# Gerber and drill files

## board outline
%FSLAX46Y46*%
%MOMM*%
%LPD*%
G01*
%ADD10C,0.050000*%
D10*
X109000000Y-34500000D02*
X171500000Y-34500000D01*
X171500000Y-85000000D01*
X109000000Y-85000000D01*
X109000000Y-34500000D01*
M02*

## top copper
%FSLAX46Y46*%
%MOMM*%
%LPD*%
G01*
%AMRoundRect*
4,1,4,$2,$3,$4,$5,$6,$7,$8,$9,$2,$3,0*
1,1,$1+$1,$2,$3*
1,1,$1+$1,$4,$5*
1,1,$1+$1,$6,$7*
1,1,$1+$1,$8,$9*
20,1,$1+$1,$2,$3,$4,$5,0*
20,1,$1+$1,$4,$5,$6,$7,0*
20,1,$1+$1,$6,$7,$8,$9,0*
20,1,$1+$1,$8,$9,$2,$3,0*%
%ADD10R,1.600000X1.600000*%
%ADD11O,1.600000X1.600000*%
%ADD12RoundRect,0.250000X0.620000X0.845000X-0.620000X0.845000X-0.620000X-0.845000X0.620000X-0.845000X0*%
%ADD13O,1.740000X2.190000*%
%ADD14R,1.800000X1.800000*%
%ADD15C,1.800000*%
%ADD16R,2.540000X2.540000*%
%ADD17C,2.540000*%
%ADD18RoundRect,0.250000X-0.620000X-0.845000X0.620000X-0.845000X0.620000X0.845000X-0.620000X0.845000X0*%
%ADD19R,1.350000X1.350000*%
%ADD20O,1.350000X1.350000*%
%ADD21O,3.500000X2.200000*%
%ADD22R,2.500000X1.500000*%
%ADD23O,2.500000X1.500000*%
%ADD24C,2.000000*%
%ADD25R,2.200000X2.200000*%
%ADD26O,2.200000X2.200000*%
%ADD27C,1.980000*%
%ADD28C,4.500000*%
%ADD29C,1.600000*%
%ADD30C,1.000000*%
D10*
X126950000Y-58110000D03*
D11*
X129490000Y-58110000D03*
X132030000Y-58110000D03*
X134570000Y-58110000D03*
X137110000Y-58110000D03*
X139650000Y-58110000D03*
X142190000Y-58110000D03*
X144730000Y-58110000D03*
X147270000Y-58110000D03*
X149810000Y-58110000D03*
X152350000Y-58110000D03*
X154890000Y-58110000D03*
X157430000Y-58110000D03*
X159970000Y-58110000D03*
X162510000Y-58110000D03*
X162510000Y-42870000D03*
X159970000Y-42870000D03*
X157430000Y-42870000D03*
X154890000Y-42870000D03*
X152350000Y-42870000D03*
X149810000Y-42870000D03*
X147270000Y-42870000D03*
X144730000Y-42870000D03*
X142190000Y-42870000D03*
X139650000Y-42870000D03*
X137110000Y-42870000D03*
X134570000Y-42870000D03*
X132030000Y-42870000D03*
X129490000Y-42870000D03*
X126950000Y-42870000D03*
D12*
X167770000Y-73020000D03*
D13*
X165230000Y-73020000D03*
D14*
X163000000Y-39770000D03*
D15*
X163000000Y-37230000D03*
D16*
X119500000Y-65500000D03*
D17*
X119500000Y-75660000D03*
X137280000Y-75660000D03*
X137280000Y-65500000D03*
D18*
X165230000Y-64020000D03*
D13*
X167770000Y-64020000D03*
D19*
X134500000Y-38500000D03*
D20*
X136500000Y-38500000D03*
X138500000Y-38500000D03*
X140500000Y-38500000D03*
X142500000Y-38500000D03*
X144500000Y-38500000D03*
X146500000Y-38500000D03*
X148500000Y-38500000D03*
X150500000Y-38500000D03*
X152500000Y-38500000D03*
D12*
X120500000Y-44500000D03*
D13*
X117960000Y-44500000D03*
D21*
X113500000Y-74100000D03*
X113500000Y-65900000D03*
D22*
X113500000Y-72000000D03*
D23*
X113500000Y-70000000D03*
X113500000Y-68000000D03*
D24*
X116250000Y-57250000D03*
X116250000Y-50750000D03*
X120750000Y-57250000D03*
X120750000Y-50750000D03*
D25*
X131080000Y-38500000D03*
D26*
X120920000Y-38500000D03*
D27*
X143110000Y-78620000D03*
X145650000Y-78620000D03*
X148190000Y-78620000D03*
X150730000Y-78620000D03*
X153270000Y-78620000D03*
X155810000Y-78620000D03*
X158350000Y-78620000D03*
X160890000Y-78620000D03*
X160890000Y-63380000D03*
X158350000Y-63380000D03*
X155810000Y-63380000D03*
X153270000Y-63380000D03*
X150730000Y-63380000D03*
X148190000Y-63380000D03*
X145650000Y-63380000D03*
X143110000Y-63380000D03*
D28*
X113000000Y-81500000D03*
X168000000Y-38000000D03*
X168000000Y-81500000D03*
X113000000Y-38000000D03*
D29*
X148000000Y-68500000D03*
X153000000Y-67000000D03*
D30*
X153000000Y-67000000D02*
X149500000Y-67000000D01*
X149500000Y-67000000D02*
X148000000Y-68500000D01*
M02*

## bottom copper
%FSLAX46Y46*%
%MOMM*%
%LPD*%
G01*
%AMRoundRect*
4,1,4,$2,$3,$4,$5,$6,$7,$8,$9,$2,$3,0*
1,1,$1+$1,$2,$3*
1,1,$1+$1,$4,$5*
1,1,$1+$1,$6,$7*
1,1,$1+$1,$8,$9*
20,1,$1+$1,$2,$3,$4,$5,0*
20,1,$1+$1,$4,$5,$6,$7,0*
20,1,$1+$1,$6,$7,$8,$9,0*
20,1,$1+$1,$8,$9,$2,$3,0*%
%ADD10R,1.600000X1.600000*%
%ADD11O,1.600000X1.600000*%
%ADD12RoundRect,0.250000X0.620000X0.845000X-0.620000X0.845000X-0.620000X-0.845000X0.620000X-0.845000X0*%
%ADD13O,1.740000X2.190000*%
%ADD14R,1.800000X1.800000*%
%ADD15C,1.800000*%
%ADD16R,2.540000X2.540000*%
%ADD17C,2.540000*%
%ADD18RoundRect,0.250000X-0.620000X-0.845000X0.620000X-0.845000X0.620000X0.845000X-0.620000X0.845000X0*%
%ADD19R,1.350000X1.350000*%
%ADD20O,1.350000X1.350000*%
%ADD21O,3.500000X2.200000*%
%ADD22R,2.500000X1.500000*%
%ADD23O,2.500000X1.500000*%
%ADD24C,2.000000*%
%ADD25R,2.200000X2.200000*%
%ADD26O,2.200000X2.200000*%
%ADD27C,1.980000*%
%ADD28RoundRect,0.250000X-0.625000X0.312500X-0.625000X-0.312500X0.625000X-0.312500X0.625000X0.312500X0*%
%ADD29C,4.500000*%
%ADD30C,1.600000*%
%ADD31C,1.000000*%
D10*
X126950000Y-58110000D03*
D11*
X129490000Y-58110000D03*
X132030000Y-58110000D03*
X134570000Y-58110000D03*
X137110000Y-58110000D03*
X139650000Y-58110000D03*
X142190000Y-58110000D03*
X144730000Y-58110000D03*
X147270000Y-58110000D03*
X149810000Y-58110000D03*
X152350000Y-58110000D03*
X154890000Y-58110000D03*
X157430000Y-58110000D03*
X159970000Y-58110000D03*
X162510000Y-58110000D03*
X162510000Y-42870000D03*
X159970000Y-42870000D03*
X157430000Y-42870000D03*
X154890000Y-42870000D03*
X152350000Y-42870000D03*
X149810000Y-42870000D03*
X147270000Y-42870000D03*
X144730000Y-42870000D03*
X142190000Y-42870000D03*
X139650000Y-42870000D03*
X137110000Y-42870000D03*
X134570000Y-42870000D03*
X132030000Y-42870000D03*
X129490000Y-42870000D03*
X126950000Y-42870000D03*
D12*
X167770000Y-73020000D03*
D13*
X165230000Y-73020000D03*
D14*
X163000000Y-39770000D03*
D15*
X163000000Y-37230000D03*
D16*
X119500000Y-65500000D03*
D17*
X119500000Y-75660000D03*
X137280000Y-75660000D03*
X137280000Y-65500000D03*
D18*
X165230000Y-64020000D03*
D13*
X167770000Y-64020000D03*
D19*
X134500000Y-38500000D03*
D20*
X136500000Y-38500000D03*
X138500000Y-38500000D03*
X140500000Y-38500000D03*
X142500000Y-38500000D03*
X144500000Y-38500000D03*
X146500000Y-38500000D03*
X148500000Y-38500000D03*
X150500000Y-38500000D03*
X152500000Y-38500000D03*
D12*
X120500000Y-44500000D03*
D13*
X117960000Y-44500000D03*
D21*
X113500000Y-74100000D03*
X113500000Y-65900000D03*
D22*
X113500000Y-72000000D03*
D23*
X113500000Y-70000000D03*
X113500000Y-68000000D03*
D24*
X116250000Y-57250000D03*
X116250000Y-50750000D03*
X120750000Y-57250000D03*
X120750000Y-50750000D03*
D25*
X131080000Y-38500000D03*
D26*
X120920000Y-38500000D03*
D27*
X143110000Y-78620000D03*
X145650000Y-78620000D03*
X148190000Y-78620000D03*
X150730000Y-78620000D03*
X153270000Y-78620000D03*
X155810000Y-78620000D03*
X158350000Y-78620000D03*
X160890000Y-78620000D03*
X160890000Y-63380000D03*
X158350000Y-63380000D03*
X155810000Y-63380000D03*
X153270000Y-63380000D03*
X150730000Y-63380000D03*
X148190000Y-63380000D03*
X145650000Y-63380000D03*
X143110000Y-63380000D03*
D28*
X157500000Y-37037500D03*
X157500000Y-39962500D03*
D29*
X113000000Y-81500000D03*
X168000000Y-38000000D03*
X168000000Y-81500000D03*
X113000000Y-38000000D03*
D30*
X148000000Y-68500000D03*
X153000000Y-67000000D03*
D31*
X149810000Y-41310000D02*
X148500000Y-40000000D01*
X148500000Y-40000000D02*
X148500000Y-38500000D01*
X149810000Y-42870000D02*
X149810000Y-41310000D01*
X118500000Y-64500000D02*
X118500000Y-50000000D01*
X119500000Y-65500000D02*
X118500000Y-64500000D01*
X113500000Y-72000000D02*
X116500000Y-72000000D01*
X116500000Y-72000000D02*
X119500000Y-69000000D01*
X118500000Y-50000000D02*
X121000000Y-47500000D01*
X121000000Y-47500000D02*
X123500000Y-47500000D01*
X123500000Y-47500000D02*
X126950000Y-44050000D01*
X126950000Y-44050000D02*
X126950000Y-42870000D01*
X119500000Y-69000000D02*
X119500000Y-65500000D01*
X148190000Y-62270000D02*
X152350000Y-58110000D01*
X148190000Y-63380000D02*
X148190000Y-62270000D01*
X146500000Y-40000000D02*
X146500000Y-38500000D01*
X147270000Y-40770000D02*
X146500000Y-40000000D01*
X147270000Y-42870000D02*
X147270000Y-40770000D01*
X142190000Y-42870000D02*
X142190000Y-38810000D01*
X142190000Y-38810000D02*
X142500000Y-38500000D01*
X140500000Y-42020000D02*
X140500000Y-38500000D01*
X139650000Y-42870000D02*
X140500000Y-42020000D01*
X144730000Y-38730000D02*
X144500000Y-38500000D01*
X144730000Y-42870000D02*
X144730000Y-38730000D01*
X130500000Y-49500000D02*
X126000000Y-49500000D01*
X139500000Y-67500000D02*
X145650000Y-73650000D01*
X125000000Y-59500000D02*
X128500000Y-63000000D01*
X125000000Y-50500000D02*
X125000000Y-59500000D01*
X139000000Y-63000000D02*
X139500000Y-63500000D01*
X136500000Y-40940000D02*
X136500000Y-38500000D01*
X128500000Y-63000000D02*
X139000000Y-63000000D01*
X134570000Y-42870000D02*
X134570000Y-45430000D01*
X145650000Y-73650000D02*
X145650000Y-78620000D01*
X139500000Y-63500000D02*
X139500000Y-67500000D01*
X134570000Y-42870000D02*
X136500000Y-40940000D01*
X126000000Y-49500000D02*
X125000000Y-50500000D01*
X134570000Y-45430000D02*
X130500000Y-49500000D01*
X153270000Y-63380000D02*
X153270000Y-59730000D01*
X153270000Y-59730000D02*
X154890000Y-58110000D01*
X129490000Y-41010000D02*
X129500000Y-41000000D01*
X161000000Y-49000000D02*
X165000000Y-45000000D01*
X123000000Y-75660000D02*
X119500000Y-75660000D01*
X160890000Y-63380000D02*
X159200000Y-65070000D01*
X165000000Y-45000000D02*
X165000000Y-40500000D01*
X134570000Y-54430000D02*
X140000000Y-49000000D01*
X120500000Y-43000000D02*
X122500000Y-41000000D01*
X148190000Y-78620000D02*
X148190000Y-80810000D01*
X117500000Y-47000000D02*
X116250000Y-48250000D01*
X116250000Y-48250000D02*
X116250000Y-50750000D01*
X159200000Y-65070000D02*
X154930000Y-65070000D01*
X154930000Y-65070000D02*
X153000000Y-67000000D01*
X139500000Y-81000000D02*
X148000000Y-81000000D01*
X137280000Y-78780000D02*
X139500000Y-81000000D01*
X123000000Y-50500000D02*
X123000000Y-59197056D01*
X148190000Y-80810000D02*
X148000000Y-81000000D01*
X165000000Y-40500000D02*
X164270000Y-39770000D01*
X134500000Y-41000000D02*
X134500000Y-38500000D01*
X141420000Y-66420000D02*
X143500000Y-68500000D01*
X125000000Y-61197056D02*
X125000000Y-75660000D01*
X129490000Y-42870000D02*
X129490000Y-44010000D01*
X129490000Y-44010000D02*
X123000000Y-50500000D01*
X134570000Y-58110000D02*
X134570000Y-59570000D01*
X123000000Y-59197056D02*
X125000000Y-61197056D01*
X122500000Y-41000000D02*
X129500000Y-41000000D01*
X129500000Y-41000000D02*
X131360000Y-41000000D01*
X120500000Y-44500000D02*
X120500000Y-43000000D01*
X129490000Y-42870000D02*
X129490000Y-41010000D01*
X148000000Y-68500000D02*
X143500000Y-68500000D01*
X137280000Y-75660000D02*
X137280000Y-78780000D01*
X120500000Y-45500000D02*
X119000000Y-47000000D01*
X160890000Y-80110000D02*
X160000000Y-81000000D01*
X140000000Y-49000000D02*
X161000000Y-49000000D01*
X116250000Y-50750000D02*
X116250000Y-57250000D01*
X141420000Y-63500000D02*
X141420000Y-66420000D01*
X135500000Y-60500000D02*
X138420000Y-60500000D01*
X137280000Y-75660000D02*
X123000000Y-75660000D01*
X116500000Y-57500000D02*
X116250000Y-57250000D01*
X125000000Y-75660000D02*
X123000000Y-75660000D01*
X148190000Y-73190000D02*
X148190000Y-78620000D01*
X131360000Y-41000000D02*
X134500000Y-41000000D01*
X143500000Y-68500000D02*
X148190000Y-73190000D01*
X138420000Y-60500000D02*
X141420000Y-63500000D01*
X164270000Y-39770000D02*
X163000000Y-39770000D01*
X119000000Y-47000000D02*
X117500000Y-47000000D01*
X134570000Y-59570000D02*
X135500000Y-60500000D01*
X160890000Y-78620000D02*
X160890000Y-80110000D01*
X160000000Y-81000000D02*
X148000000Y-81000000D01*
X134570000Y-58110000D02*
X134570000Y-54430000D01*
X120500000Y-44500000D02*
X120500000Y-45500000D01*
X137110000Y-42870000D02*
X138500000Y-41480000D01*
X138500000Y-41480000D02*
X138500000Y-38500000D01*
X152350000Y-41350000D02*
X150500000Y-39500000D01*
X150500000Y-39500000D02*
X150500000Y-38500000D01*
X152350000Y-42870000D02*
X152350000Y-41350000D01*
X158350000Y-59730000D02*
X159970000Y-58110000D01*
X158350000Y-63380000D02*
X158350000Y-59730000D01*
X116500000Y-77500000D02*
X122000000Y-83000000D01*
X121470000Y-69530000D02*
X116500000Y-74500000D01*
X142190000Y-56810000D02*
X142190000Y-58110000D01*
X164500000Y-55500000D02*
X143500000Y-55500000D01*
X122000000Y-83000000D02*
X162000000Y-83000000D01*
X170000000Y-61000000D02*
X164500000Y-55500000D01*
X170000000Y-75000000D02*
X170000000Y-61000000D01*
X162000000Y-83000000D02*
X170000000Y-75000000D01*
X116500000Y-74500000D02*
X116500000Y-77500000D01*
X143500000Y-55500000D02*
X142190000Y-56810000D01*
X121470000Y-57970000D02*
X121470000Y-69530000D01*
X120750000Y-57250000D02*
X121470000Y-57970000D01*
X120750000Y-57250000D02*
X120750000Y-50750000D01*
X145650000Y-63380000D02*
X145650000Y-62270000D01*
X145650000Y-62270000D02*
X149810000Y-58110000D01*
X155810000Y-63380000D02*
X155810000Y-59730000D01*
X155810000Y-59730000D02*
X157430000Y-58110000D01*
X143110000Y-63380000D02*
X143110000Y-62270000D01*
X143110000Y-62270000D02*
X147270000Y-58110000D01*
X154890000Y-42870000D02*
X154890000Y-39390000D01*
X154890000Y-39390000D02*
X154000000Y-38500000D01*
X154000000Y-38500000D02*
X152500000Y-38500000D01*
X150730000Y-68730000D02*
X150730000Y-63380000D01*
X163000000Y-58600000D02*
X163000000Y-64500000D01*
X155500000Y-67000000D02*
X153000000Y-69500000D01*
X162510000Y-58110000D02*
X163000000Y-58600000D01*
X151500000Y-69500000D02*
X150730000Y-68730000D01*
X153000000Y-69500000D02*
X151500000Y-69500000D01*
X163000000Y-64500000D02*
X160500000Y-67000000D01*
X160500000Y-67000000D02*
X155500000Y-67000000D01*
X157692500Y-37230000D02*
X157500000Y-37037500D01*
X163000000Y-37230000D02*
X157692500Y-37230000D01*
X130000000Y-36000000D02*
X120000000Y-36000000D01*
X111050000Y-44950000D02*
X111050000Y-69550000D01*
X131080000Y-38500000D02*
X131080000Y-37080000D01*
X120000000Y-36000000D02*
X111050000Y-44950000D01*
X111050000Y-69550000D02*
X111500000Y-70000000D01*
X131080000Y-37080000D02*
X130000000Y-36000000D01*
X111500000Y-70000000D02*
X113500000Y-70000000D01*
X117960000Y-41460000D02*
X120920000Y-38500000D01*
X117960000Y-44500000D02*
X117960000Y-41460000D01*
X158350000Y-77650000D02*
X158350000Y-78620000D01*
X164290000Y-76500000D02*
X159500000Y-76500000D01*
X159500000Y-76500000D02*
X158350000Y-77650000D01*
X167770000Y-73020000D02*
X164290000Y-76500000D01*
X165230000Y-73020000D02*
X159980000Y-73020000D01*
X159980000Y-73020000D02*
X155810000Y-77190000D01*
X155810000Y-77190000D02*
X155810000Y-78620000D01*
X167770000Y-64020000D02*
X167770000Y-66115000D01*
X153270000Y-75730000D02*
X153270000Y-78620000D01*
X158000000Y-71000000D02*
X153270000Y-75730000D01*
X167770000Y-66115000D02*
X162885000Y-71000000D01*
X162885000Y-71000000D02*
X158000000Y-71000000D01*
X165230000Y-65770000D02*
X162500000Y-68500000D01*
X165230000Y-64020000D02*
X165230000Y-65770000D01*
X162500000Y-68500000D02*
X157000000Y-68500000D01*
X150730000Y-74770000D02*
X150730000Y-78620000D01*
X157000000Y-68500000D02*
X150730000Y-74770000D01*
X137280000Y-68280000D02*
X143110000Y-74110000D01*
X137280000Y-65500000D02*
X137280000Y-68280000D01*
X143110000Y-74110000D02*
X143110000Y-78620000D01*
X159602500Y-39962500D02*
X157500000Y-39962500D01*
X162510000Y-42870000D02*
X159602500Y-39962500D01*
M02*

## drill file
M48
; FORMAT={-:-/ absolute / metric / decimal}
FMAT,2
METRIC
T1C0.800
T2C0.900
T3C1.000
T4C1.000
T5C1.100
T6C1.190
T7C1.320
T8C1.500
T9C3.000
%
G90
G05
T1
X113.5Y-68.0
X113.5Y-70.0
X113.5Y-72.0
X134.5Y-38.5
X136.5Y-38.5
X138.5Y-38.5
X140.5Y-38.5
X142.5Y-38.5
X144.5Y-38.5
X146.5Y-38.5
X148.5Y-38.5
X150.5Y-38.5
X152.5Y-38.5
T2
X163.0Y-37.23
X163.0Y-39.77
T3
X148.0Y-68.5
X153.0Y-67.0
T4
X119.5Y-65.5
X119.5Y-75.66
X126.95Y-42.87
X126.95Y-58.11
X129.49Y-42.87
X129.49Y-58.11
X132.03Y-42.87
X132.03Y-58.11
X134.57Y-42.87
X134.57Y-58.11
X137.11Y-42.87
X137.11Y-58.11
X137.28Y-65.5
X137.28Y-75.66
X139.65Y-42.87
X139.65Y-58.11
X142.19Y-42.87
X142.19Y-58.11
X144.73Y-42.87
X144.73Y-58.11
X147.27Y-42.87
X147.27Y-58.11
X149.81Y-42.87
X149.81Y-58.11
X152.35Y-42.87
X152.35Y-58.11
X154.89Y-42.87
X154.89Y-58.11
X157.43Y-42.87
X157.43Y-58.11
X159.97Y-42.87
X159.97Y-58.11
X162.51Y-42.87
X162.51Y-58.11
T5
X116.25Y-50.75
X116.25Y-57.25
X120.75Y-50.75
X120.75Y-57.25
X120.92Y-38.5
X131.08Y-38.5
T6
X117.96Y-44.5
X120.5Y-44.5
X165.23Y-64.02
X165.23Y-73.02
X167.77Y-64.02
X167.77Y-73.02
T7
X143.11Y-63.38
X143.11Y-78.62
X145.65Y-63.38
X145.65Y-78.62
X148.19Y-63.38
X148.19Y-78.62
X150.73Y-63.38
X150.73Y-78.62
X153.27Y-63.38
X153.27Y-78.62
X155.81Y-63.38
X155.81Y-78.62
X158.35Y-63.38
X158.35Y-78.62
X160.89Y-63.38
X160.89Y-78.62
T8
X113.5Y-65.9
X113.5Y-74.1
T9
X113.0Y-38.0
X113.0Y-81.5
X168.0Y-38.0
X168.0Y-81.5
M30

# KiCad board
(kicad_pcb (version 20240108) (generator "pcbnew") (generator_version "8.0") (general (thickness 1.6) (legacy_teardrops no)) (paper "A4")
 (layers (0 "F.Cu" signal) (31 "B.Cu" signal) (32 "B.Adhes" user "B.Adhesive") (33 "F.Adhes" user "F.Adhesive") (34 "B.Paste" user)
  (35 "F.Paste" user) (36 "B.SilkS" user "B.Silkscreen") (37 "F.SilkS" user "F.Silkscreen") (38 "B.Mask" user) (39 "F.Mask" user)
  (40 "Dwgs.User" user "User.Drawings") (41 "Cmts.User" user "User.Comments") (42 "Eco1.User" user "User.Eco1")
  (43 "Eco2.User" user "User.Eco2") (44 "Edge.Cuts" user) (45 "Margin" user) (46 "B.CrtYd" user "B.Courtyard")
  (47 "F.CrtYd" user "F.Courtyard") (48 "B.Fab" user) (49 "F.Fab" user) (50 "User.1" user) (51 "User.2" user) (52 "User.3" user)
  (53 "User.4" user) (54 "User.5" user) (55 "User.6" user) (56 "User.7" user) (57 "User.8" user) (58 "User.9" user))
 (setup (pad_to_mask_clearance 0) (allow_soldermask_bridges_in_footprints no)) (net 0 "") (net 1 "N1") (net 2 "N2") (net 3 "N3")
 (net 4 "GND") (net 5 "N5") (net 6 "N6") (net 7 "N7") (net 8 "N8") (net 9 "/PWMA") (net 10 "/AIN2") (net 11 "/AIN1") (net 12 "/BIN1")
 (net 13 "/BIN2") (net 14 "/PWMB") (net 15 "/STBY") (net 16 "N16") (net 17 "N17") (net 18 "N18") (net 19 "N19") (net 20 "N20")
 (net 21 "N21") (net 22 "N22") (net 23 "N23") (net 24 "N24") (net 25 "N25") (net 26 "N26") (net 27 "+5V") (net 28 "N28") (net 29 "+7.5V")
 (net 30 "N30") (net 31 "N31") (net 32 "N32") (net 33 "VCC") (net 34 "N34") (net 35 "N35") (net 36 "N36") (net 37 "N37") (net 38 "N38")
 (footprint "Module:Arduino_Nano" (layer "F.Cu") (at 126.95 58.11 90)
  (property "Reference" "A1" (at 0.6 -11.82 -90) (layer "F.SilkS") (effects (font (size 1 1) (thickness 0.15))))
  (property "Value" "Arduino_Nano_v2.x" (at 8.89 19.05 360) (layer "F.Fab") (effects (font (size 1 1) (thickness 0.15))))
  (pad "1" thru_hole rect (at 0 0 90) (size 1.6 1.6) (drill 1) (layers "*.Cu" "*.Mask") (remove_unused_layers no) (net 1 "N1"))
  (pad "2" thru_hole oval (at 0 2.54 90) (size 1.6 1.6) (drill 1) (layers "*.Cu" "*.Mask") (remove_unused_layers no) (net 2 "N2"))
  (pad "3" thru_hole oval (at 0 5.08 90) (size 1.6 1.6) (drill 1) (layers "*.Cu" "*.Mask") (remove_unused_layers no) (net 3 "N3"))
  (pad "4" thru_hole oval (at 0 7.62 90) (size 1.6 1.6) (drill 1) (layers "*.Cu" "*.Mask") (remove_unused_layers no) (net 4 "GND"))
  (pad "5" thru_hole oval (at 0 10.16 90) (size 1.6 1.6) (drill 1) (layers "*.Cu" "*.Mask") (remove_unused_layers no) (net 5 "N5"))
  (pad "6" thru_hole oval (at 0 12.7 90) (size 1.6 1.6) (drill 1) (layers "*.Cu" "*.Mask") (remove_unused_layers no) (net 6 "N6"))
  (pad "7" thru_hole oval (at 0 15.24 90) (size 1.6 1.6) (drill 1) (layers "*.Cu" "*.Mask") (remove_unused_layers no) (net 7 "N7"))
  (pad "8" thru_hole oval (at 0 17.78 90) (size 1.6 1.6) (drill 1) (layers "*.Cu" "*.Mask") (remove_unused_layers no) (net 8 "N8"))
  (pad "9" thru_hole oval (at 0 20.32 90) (size 1.6 1.6) (drill 1) (layers "*.Cu" "*.Mask") (remove_unused_layers no) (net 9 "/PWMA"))
  (pad "10" thru_hole oval (at 0 22.86 90) (size 1.6 1.6) (drill 1) (layers "*.Cu" "*.Mask") (remove_unused_layers no) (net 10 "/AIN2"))
  (pad "11" thru_hole oval (at 0 25.4 90) (size 1.6 1.6) (drill 1) (layers "*.Cu" "*.Mask") (remove_unused_layers no) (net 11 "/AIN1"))
  (pad "12" thru_hole oval (at 0 27.94 90) (size 1.6 1.6) (drill 1) (layers "*.Cu" "*.Mask") (remove_unused_layers no) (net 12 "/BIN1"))
  (pad "13" thru_hole oval (at 0 30.48 90) (size 1.6 1.6) (drill 1) (layers "*.Cu" "*.Mask") (remove_unused_layers no) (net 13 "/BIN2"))
  (pad "14" thru_hole oval (at 0 33.02 90) (size 1.6 1.6) (drill 1) (layers "*.Cu" "*.Mask") (remove_unused_layers no) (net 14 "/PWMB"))
  (pad "15" thru_hole oval (at 0 35.56 90) (size 1.6 1.6) (drill 1) (layers "*.Cu" "*.Mask") (remove_unused_layers no) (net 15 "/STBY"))
  (pad "16" thru_hole oval (at 15.24 35.56 90) (size 1.6 1.6) (drill 1) (layers "*.Cu" "*.Mask") (remove_unused_layers no) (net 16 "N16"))
  (pad "17" thru_hole oval (at 15.24 33.02 90) (size 1.6 1.6) (drill 1) (layers "*.Cu" "*.Mask") (remove_unused_layers no) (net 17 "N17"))
  (pad "18" thru_hole oval (at 15.24 30.48 90) (size 1.6 1.6) (drill 1) (layers "*.Cu" "*.Mask") (remove_unused_layers no) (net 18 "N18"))
  (pad "19" thru_hole oval (at 15.24 27.94 90) (size 1.6 1.6) (drill 1) (layers "*.Cu" "*.Mask") (remove_unused_layers no) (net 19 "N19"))
  (pad "20" thru_hole oval (at 15.24 25.4 90) (size 1.6 1.6) (drill 1) (layers "*.Cu" "*.Mask") (remove_unused_layers no) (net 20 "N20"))
  (pad "21" thru_hole oval (at 15.24 22.86 90) (size 1.6 1.6) (drill 1) (layers "*.Cu" "*.Mask") (remove_unused_layers no) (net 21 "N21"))
  (pad "22" thru_hole oval (at 15.24 20.32 90) (size 1.6 1.6) (drill 1) (layers "*.Cu" "*.Mask") (remove_unused_layers no) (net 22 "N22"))
  (pad "23" thru_hole oval (at 15.24 17.78 90) (size 1.6 1.6) (drill 1) (layers "*.Cu" "*.Mask") (remove_unused_layers no) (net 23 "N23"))
  (pad "24" thru_hole oval (at 15.24 15.24 90) (size 1.6 1.6) (drill 1) (layers "*.Cu" "*.Mask") (remove_unused_layers no) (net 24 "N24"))
  (pad "25" thru_hole oval (at 15.24 12.7 90) (size 1.6 1.6) (drill 1) (layers "*.Cu" "*.Mask") (remove_unused_layers no) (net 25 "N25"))
  (pad "26" thru_hole oval (at 15.24 10.16 90) (size 1.6 1.6) (drill 1) (layers "*.Cu" "*.Mask") (remove_unused_layers no) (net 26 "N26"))
  (pad "27" thru_hole oval (at 15.24 7.62 90) (size 1.6 1.6) (drill 1) (layers "*.Cu" "*.Mask") (remove_unused_layers no) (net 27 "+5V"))
  (pad "28" thru_hole oval (at 15.24 5.08 90) (size 1.6 1.6) (drill 1) (layers "*.Cu" "*.Mask") (remove_unused_layers no) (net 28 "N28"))
  (pad "29" thru_hole oval (at 15.24 2.54 90) (size 1.6 1.6) (drill 1) (layers "*.Cu" "*.Mask") (remove_unused_layers no) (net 4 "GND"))
  (pad "30" thru_hole oval (at 15.24 0 90) (size 1.6 1.6) (drill 1) (layers "*.Cu" "*.Mask") (remove_unused_layers no) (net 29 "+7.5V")))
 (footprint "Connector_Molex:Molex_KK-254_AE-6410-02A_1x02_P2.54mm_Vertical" (layer "F.Cu") (at 167.77 73.02 180)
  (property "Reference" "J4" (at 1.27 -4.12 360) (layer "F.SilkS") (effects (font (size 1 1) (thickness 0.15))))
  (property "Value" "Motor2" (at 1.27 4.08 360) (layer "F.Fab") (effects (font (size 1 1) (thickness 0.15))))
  (pad "1" thru_hole roundrect (at 0 0 180) (size 1.74 2.19) (drill 1.19) (layers "*.Cu" "*.Mask") (remove_unused_layers no)
   (roundrect_rratio 0.143678) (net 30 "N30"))
  (pad "2" thru_hole oval (at 2.54 0 180) (size 1.74 2.19) (drill 1.19) (layers "*.Cu" "*.Mask") (remove_unused_layers no) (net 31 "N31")))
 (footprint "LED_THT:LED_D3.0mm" (layer "F.Cu") (at 163 39.77 90)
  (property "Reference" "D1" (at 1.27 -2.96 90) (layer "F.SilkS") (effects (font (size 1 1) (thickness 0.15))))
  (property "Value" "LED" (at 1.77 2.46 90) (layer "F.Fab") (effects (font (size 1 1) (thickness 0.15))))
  (pad "1" thru_hole rect (at 0 0 90) (size 1.8 1.8) (drill 0.9) (layers "*.Cu" "*.Mask") (remove_unused_layers no) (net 4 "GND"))
  (pad "2" thru_hole circle (at 2.54 0 90) (size 1.8 1.8) (drill 0.9) (layers "*.Cu" "*.Mask") (remove_unused_layers no) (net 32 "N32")))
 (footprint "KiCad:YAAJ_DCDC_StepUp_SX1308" (layer "F.Cu") (at 119.5 65.5)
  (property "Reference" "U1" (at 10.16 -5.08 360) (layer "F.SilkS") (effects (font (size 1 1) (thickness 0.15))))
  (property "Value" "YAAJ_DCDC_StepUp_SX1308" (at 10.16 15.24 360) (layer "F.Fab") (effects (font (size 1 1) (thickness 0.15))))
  (pad "1" thru_hole rect (at 0 0) (size 2.54 2.54) (drill 1) (layers "*.Cu" "*.Mask") (remove_unused_layers no) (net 29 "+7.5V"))
  (pad "2" thru_hole circle (at 0 10.16) (size 2.54 2.54) (drill 1) (layers "*.Cu" "*.Mask") (remove_unused_layers no) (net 4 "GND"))
  (pad "3" thru_hole circle (at 17.78 10.16) (size 2.54 2.54) (drill 1) (layers "*.Cu" "*.Mask") (remove_unused_layers no) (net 4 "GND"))
  (pad "4" thru_hole circle (at 17.78 0) (size 2.54 2.54) (drill 1) (layers "*.Cu" "*.Mask") (remove_unused_layers no) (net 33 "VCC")))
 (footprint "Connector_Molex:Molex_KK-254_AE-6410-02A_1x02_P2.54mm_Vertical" (layer "F.Cu") (at 165.23 64.02)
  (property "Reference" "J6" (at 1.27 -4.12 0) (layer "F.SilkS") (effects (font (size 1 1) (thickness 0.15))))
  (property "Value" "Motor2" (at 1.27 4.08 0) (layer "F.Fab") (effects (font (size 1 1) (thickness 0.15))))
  (pad "1" thru_hole roundrect (at 0 0) (size 1.74 2.19) (drill 1.19) (layers "*.Cu" "*.Mask") (remove_unused_layers no)
   (roundrect_rratio 0.143678) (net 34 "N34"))
  (pad "2" thru_hole oval (at 2.54 0) (size 1.74 2.19) (drill 1.19) (layers "*.Cu" "*.Mask") (remove_unused_layers no) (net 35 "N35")))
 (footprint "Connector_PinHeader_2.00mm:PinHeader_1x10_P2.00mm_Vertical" (layer "F.Cu") (at 134.5 38.5 90)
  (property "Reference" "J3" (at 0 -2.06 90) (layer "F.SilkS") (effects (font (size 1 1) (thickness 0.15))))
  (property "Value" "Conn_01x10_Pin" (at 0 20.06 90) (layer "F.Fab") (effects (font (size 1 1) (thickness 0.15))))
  (pad "1" thru_hole rect (at 0 0 90) (size 1.35 1.35) (drill 0.8) (layers "*.Cu" "*.Mask") (remove_unused_layers no) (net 4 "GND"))
  (pad "2" thru_hole oval (at 0 2 90) (size 1.35 1.35) (drill 0.8) (layers "*.Cu" "*.Mask") (remove_unused_layers no) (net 27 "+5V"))
  (pad "3" thru_hole oval (at 0 4 90) (size 1.35 1.35) (drill 0.8) (layers "*.Cu" "*.Mask") (remove_unused_layers no) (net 26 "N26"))
  (pad "4" thru_hole oval (at 0 6 90) (size 1.35 1.35) (drill 0.8) (layers "*.Cu" "*.Mask") (remove_unused_layers no) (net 25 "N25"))
  (pad "5" thru_hole oval (at 0 8 90) (size 1.35 1.35) (drill 0.8) (layers "*.Cu" "*.Mask") (remove_unused_layers no) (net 24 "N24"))
  (pad "6" thru_hole oval (at 0 10 90) (size 1.35 1.35) (drill 0.8) (layers "*.Cu" "*.Mask") (remove_unused_layers no) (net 23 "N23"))
  (pad "7" thru_hole oval (at 0 12 90) (size 1.35 1.35) (drill 0.8) (layers "*.Cu" "*.Mask") (remove_unused_layers no) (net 22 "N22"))
  (pad "8" thru_hole oval (at 0 14 90) (size 1.35 1.35) (drill 0.8) (layers "*.Cu" "*.Mask") (remove_unused_layers no) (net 21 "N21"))
  (pad "9" thru_hole oval (at 0 16 90) (size 1.35 1.35) (drill 0.8) (layers "*.Cu" "*.Mask") (remove_unused_layers no) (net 20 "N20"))
  (pad "10" thru_hole oval (at 0 18 90) (size 1.35 1.35) (drill 0.8) (layers "*.Cu" "*.Mask") (remove_unused_layers no) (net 19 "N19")))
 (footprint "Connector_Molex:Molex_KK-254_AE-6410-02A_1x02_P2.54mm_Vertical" (layer "F.Cu") (at 120.5 44.5 180)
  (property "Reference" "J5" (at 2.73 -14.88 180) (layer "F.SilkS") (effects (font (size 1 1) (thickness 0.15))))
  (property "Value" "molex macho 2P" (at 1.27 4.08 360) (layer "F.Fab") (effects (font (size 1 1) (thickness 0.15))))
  (pad "1" thru_hole roundrect (at 0 0 180) (size 1.74 2.19) (drill 1.19) (layers "*.Cu" "*.Mask") (remove_unused_layers no)
   (roundrect_rratio 0.143678) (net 4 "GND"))
  (pad "2" thru_hole oval (at 2.54 0 180) (size 1.74 2.19) (drill 1.19) (layers "*.Cu" "*.Mask") (remove_unused_layers no) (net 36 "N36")))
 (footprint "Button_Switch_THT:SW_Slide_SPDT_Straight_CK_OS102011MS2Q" (layer "F.Cu") (at 113.5 72 90)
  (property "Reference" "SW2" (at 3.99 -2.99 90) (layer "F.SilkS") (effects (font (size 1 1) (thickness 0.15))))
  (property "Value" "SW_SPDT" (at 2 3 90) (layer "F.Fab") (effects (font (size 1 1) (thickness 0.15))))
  (pad "" thru_hole oval (at -2.1 0 90) (size 2.2 3.5) (drill 1.5) (layers "*.Cu" "*.Mask") (remove_unused_layers no))
  (pad "" thru_hole oval (at 6.1 0 90) (size 2.2 3.5) (drill 1.5) (layers "*.Cu" "*.Mask") (remove_unused_layers no))
  (pad "1" thru_hole rect (at 0 0 90) (size 1.5 2.5) (drill 0.8) (layers "*.Cu" "*.Mask") (remove_unused_layers no) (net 29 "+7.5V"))
  (pad "2" thru_hole oval (at 2 0 90) (size 1.5 2.5) (drill 0.8) (layers "*.Cu" "*.Mask") (remove_unused_layers no) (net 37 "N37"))
  (pad "3" thru_hole oval (at 4 0 90) (size 1.5 2.5) (drill 0.8) (layers "*.Cu" "*.Mask") (remove_unused_layers no) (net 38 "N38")))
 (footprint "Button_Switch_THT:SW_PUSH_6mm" (layer "F.Cu") (at 116.25 57.25 90)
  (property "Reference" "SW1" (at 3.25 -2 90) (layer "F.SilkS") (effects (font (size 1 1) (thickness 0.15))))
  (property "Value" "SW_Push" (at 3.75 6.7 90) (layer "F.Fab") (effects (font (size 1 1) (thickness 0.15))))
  (pad "1" thru_hole circle (at 0 0 180) (size 2 2) (drill 1.1) (layers "*.Cu" "*.Mask") (remove_unused_layers no) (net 4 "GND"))
  (pad "1" thru_hole circle (at 6.5 0 180) (size 2 2) (drill 1.1) (layers "*.Cu" "*.Mask") (remove_unused_layers no) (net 4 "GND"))
  (pad "2" thru_hole circle (at 0 4.5 180) (size 2 2) (drill 1.1) (layers "*.Cu" "*.Mask") (remove_unused_layers no) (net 7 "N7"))
  (pad "2" thru_hole circle (at 6.5 4.5 180) (size 2 2) (drill 1.1) (layers "*.Cu" "*.Mask") (remove_unused_layers no) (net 7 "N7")))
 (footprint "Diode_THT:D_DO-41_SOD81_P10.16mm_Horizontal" (layer "F.Cu") (at 131.08 38.5 180)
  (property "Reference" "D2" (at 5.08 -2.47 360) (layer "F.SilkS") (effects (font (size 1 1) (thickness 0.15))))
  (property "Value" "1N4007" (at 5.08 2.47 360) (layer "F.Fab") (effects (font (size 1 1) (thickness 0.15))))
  (pad "1" thru_hole rect (at 0 0 180) (size 2.2 2.2) (drill 1.1) (layers "*.Cu" "*.Mask") (remove_unused_layers no) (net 37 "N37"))
  (pad "2" thru_hole oval (at 10.16 0 180) (size 2.2 2.2) (drill 1.1) (layers "*.Cu" "*.Mask") (remove_unused_layers no) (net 36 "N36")))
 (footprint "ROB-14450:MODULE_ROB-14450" (layer "F.Cu") (at 152 71 90)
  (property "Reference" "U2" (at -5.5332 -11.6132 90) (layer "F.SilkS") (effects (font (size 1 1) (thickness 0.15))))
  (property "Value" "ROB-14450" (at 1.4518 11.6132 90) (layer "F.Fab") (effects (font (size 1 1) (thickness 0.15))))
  (pad "1" thru_hole circle (at -7.62 -8.89 90) (size 1.98 1.98) (drill 1.32) (layers "*.Cu" "*.Mask") (remove_unused_layers no)
   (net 33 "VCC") (solder_mask_margin 0.102))
  (pad "2" thru_hole circle (at -7.62 -6.35 90) (size 1.98 1.98) (drill 1.32) (layers "*.Cu" "*.Mask") (remove_unused_layers no)
   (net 27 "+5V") (solder_mask_margin 0.102))
  (pad "3" thru_hole circle (at -7.62 -3.81 90) (size 1.98 1.98) (drill 1.32) (layers "*.Cu" "*.Mask") (remove_unused_layers no)
   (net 4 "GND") (solder_mask_margin 0.102))
  (pad "4" thru_hole circle (at -7.62 -1.27 90) (size 1.98 1.98) (drill 1.32) (layers "*.Cu" "*.Mask") (remove_unused_layers no)
   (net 34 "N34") (solder_mask_margin 0.102))
  (pad "5" thru_hole circle (at -7.62 1.27 90) (size 1.98 1.98) (drill 1.32) (layers "*.Cu" "*.Mask") (remove_unused_layers no)
   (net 35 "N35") (solder_mask_margin 0.102))
  (pad "6" thru_hole circle (at -7.62 3.81 90) (size 1.98 1.98) (drill 1.32) (layers "*.Cu" "*.Mask") (remove_unused_layers no)
   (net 31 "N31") (solder_mask_margin 0.102))
  (pad "7" thru_hole circle (at -7.62 6.35 90) (size 1.98 1.98) (drill 1.32) (layers "*.Cu" "*.Mask") (remove_unused_layers no)
   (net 30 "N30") (solder_mask_margin 0.102))
  (pad "8" thru_hole circle (at -7.62 8.89 90) (size 1.98 1.98) (drill 1.32) (layers "*.Cu" "*.Mask") (remove_unused_layers no)
   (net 4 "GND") (solder_mask_margin 0.102))
  (pad "9" thru_hole circle (at 7.62 8.89 90) (size 1.98 1.98) (drill 1.32) (layers "*.Cu" "*.Mask") (remove_unused_layers no) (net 4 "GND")
   (solder_mask_margin 0.102))
  (pad "10" thru_hole circle (at 7.62 6.35 90) (size 1.98 1.98) (drill 1.32) (layers "*.Cu" "*.Mask") (remove_unused_layers no)
   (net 14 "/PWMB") (solder_mask_margin 0.102))
  (pad "11" thru_hole circle (at 7.62 3.81 90) (size 1.98 1.98) (drill 1.32) (layers "*.Cu" "*.Mask") (remove_unused_layers no)
   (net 13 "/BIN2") (solder_mask_margin 0.102))
  (pad "12" thru_hole circle (at 7.62 1.27 90) (size 1.98 1.98) (drill 1.32) (layers "*.Cu" "*.Mask") (remove_unused_layers no)
   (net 12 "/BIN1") (solder_mask_margin 0.102))
  (pad "13" thru_hole circle (at 7.62 -1.27 90) (size 1.98 1.98) (drill 1.32) (layers "*.Cu" "*.Mask") (remove_unused_layers no)
   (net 15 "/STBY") (solder_mask_margin 0.102))
  (pad "14" thru_hole circle (at 7.62 -3.81 90) (size 1.98 1.98) (drill 1.32) (layers "*.Cu" "*.Mask") (remove_unused_layers no)
   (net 11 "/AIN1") (solder_mask_margin 0.102))
  (pad "15" thru_hole circle (at 7.62 -6.35 90) (size 1.98 1.98) (drill 1.32) (layers "*.Cu" "*.Mask") (remove_unused_layers no)
   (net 10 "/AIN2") (solder_mask_margin 0.102))
  (pad "16" thru_hole circle (at 7.62 -8.89 90) (size 1.98 1.98) (drill 1.32) (layers "*.Cu" "*.Mask") (remove_unused_layers no)
   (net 9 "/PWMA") (solder_mask_margin 0.102)))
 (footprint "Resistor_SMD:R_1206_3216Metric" (layer "B.Cu") (at 157.5 38.5 -90)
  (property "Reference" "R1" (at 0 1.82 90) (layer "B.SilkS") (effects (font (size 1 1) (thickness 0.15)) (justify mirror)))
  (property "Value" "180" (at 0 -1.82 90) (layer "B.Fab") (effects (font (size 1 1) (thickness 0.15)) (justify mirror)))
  (pad "1" smd roundrect (at -1.4625 0 270) (size 1.125 1.75) (layers "B.Cu" "B.Paste" "B.Mask") (roundrect_rratio 0.222222) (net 32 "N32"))
  (pad "2" smd roundrect (at 1.4625 0 270) (size 1.125 1.75) (layers "B.Cu" "B.Paste" "B.Mask") (roundrect_rratio 0.222222) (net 16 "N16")))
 (gr_rect (start 109 34.5) (end 171.5 85) (stroke (width 0.05) (type default)) (fill none) (layer "Edge.Cuts"))
 (via (at 113 81.5) (size 4.5) (drill 3) (layers "F.Cu" "B.Cu") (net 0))
 (via (at 168 38) (size 4.5) (drill 3) (layers "F.Cu" "B.Cu") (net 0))
 (via (at 168 81.5) (size 4.5) (drill 3) (layers "F.Cu" "B.Cu") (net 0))
 (via (at 113 38) (size 4.5) (drill 3) (layers "F.Cu" "B.Cu") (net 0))
 (segment (start 149.81 41.31) (end 148.5 40) (width 1) (layer "B.Cu") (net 21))
 (segment (start 148.5 40) (end 148.5 38.5) (width 1) (layer "B.Cu") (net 21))
 (segment (start 149.81 42.87) (end 149.81 41.31) (width 1) (layer "B.Cu") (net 21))
 (segment (start 118.5 64.5) (end 118.5 50) (width 1) (layer "B.Cu") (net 29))
 (segment (start 119.5 65.5) (end 118.5 64.5) (width 1) (layer "B.Cu") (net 29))
 (segment (start 113.5 72) (end 116.5 72) (width 1) (layer "B.Cu") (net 29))
 (segment (start 116.5 72) (end 119.5 69) (width 1) (layer "B.Cu") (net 29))
 (segment (start 118.5 50) (end 121 47.5) (width 1) (layer "B.Cu") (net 29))
 (segment (start 121 47.5) (end 123.5 47.5) (width 1) (layer "B.Cu") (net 29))
 (segment (start 123.5 47.5) (end 126.95 44.05) (width 1) (layer "B.Cu") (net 29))
 (segment (start 126.95 44.05) (end 126.95 42.87) (width 1) (layer "B.Cu") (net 29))
 (segment (start 119.5 69) (end 119.5 65.5) (width 1) (layer "B.Cu") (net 29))
 (segment (start 148.19 62.27) (end 152.35 58.11) (width 1) (layer "B.Cu") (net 11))
 (segment (start 148.19 63.38) (end 148.19 62.27) (width 1) (layer "B.Cu") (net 11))
 (segment (start 146.5 40) (end 146.5 38.5) (width 1) (layer "B.Cu") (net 22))
 (segment (start 147.27 40.77) (end 146.5 40) (width 1) (layer "B.Cu") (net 22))
 (segment (start 147.27 42.87) (end 147.27 40.77) (width 1) (layer "B.Cu") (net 22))
 (segment (start 142.19 42.87) (end 142.19 38.81) (width 1) (layer "B.Cu") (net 24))
 (segment (start 142.19 38.81) (end 142.5 38.5) (width 1) (layer "B.Cu") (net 24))
 (segment (start 140.5 42.02) (end 140.5 38.5) (width 1) (layer "B.Cu") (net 25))
 (segment (start 139.65 42.87) (end 140.5 42.02) (width 1) (layer "B.Cu") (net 25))
 (segment (start 144.73 38.73) (end 144.5 38.5) (width 1) (layer "B.Cu") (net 23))
 (segment (start 144.73 42.87) (end 144.73 38.73) (width 1) (layer "B.Cu") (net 23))
 (segment (start 130.5 49.5) (end 126 49.5) (width 1) (layer "B.Cu") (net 27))
 (segment (start 139.5 67.5) (end 145.65 73.65) (width 1) (layer "B.Cu") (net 27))
 (segment (start 125 59.5) (end 128.5 63) (width 1) (layer "B.Cu") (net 27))
 (segment (start 125 50.5) (end 125 59.5) (width 1) (layer "B.Cu") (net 27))
 (segment (start 139 63) (end 139.5 63.5) (width 1) (layer "B.Cu") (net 27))
 (segment (start 136.5 40.94) (end 136.5 38.5) (width 1) (layer "B.Cu") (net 27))
 (segment (start 128.5 63) (end 139 63) (width 1) (layer "B.Cu") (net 27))
 (segment (start 134.57 42.87) (end 134.57 45.43) (width 1) (layer "B.Cu") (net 27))
 (segment (start 145.65 73.65) (end 145.65 78.62) (width 1) (layer "B.Cu") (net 27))
 (segment (start 139.5 63.5) (end 139.5 67.5) (width 1) (layer "B.Cu") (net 27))
 (segment (start 134.57 42.87) (end 136.5 40.94) (width 1) (layer "B.Cu") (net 27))
 (segment (start 126 49.5) (end 125 50.5) (width 1) (layer "B.Cu") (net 27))
 (segment (start 134.57 45.43) (end 130.5 49.5) (width 1) (layer "B.Cu") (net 27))
 (segment (start 153.27 63.38) (end 153.27 59.73) (width 1) (layer "B.Cu") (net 12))
 (segment (start 153.27 59.73) (end 154.89 58.11) (width 1) (layer "B.Cu") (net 12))
 (segment (start 153 67) (end 149.5 67) (width 1) (layer "F.Cu") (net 4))
 (segment (start 149.5 67) (end 148 68.5) (width 1) (layer "F.Cu") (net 4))
 (via (at 148 68.5) (size 1.6) (drill 1) (layers "F.Cu" "B.Cu") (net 4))
 (via (at 153 67) (size 1.6) (drill 1) (layers "F.Cu" "B.Cu") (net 4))
 (segment (start 129.49 41.01) (end 129.5 41) (width 1) (layer "B.Cu") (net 4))
 (segment (start 161 49) (end 165 45) (width 1) (layer "B.Cu") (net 4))
 (segment (start 123 75.66) (end 119.5 75.66) (width 1) (layer "B.Cu") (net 4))
 (segment (start 160.89 63.38) (end 159.2 65.07) (width 1) (layer "B.Cu") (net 4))
 (segment (start 165 45) (end 165 40.5) (width 1) (layer "B.Cu") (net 4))
 (segment (start 134.57 54.43) (end 140 49) (width 1) (layer "B.Cu") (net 4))
 (segment (start 120.5 43) (end 122.5 41) (width 1) (layer "B.Cu") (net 4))
 (segment (start 148.19 78.62) (end 148.19 80.81) (width 1) (layer "B.Cu") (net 4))
 (segment (start 117.5 47) (end 116.25 48.25) (width 1) (layer "B.Cu") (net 4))
 (segment (start 116.25 48.25) (end 116.25 50.75) (width 1) (layer "B.Cu") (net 4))
 (segment (start 159.2 65.07) (end 154.93 65.07) (width 1) (layer "B.Cu") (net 4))
 (segment (start 154.93 65.07) (end 153 67) (width 1) (layer "B.Cu") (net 4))
 (segment (start 139.5 81) (end 148 81) (width 1) (layer "B.Cu") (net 4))
 (segment (start 137.28 78.78) (end 139.5 81) (width 1) (layer "B.Cu") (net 4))
 (segment (start 123 50.5) (end 123 59.197056) (width 1) (layer "B.Cu") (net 4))
 (segment (start 148.19 80.81) (end 148 81) (width 1) (layer "B.Cu") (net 4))
 (segment (start 165 40.5) (end 164.27 39.77) (width 1) (layer "B.Cu") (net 4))
 (segment (start 134.5 41) (end 134.5 38.5) (width 1) (layer "B.Cu") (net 4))
 (segment (start 141.42 66.42) (end 143.5 68.5) (width 1) (layer "B.Cu") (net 4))
 (segment (start 125 61.197056) (end 125 75.66) (width 1) (layer "B.Cu") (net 4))
 (segment (start 129.49 42.87) (end 129.49 44.01) (width 1) (layer "B.Cu") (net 4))
 (segment (start 129.49 44.01) (end 123 50.5) (width 1) (layer "B.Cu") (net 4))
 (segment (start 134.57 58.11) (end 134.57 59.57) (width 1) (layer "B.Cu") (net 4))
 (segment (start 123 59.197056) (end 125 61.197056) (width 1) (layer "B.Cu") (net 4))
 (segment (start 122.5 41) (end 129.5 41) (width 1) (layer "B.Cu") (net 4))
 (segment (start 129.5 41) (end 131.36 41) (width 1) (layer "B.Cu") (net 4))
 (segment (start 120.5 44.5) (end 120.5 43) (width 1) (layer "B.Cu") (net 4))
 (segment (start 129.49 42.87) (end 129.49 41.01) (width 1) (layer "B.Cu") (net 4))
 (segment (start 148 68.5) (end 143.5 68.5) (width 1) (layer "B.Cu") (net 4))
 (segment (start 137.28 75.66) (end 137.28 78.78) (width 1) (layer "B.Cu") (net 4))
 (segment (start 120.5 45.5) (end 119 47) (width 1) (layer "B.Cu") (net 4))
 (segment (start 160.89 80.11) (end 160 81) (width 1) (layer "B.Cu") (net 4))
 (segment (start 140 49) (end 161 49) (width 1) (layer "B.Cu") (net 4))
 (segment (start 116.25 50.75) (end 116.25 57.25) (width 1) (layer "B.Cu") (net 4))
 (segment (start 141.42 63.5) (end 141.42 66.42) (width 1) (layer "B.Cu") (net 4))
 (segment (start 135.5 60.5) (end 138.42 60.5) (width 1) (layer "B.Cu") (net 4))
 (segment (start 137.28 75.66) (end 123 75.66) (width 1) (layer "B.Cu") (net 4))
 (segment (start 116.5 57.5) (end 116.25 57.25) (width 1) (layer "B.Cu") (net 4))
 (segment (start 125 75.66) (end 123 75.66) (width 1) (layer "B.Cu") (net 4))
 (segment (start 148.19 73.19) (end 148.19 78.62) (width 1) (layer "B.Cu") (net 4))
 (segment (start 131.36 41) (end 134.5 41) (width 1) (layer "B.Cu") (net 4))
 (segment (start 143.5 68.5) (end 148.19 73.19) (width 1) (layer "B.Cu") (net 4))
 (segment (start 138.42 60.5) (end 141.42 63.5) (width 1) (layer "B.Cu") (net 4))
 (segment (start 164.27 39.77) (end 163 39.77) (width 1) (layer "B.Cu") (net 4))
 (segment (start 119 47) (end 117.5 47) (width 1) (layer "B.Cu") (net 4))
 (segment (start 134.57 59.57) (end 135.5 60.5) (width 1) (layer "B.Cu") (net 4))
 (segment (start 160.89 78.62) (end 160.89 80.11) (width 1) (layer "B.Cu") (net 4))
 (segment (start 160 81) (end 148 81) (width 1) (layer "B.Cu") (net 4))
 (segment (start 134.57 58.11) (end 134.57 54.43) (width 1) (layer "B.Cu") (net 4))
 (segment (start 120.5 44.5) (end 120.5 45.5) (width 1) (layer "B.Cu") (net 4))
 (segment (start 137.11 42.87) (end 138.5 41.48) (width 1) (layer "B.Cu") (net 26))
 (segment (start 138.5 41.48) (end 138.5 38.5) (width 1) (layer "B.Cu") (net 26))
 (segment (start 152.35 41.35) (end 150.5 39.5) (width 1) (layer "B.Cu") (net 20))
 (segment (start 150.5 39.5) (end 150.5 38.5) (width 1) (layer "B.Cu") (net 20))
 (segment (start 152.35 42.87) (end 152.35 41.35) (width 1) (layer "B.Cu") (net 20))
 (segment (start 158.35 59.73) (end 159.97 58.11) (width 1) (layer "B.Cu") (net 14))
 (segment (start 158.35 63.38) (end 158.35 59.73) (width 1) (layer "B.Cu") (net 14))
 (segment (start 116.5 77.5) (end 122 83) (width 1) (layer "B.Cu") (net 7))
 (segment (start 121.47 69.53) (end 116.5 74.5) (width 1) (layer "B.Cu") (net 7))
 (segment (start 142.19 56.81) (end 142.19 58.11) (width 1) (layer "B.Cu") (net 7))
 (segment (start 164.5 55.5) (end 143.5 55.5) (width 1) (layer "B.Cu") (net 7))
 (segment (start 122 83) (end 162 83) (width 1) (layer "B.Cu") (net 7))
 (segment (start 170 61) (end 164.5 55.5) (width 1) (layer "B.Cu") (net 7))
 (segment (start 170 75) (end 170 61) (width 1) (layer "B.Cu") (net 7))
 (segment (start 162 83) (end 170 75) (width 1) (layer "B.Cu") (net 7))
 (segment (start 116.5 74.5) (end 116.5 77.5) (width 1) (layer "B.Cu") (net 7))
 (segment (start 143.5 55.5) (end 142.19 56.81) (width 1) (layer "B.Cu") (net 7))
 (segment (start 121.47 57.97) (end 121.47 69.53) (width 1) (layer "B.Cu") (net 7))
 (segment (start 120.75 57.25) (end 121.47 57.97) (width 1) (layer "B.Cu") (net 7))
 (segment (start 120.75 57.25) (end 120.75 50.75) (width 1) (layer "B.Cu") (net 7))
 (segment (start 145.65 63.38) (end 145.65 62.27) (width 1) (layer "B.Cu") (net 10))
 (segment (start 145.65 62.27) (end 149.81 58.11) (width 1) (layer "B.Cu") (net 10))
 (segment (start 155.81 63.38) (end 155.81 59.73) (width 1) (layer "B.Cu") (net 13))
 (segment (start 155.81 59.73) (end 157.43 58.11) (width 1) (layer "B.Cu") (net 13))
 (segment (start 143.11 63.38) (end 143.11 62.27) (width 1) (layer "B.Cu") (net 9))
 (segment (start 143.11 62.27) (end 147.27 58.11) (width 1) (layer "B.Cu") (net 9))
 (segment (start 154.89 42.87) (end 154.89 39.39) (width 1) (layer "B.Cu") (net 19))
 (segment (start 154.89 39.39) (end 154 38.5) (width 1) (layer "B.Cu") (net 19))
 (segment (start 154 38.5) (end 152.5 38.5) (width 1) (layer "B.Cu") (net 19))
 (segment (start 150.73 68.73) (end 150.73 63.38) (width 1) (layer "B.Cu") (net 15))
 (segment (start 163 58.6) (end 163 64.5) (width 1) (layer "B.Cu") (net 15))
 (segment (start 155.5 67) (end 153 69.5) (width 1) (layer "B.Cu") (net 15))
 (segment (start 162.51 58.11) (end 163 58.6) (width 1) (layer "B.Cu") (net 15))
 (segment (start 151.5 69.5) (end 150.73 68.73) (width 1) (layer "B.Cu") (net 15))
 (segment (start 153 69.5) (end 151.5 69.5) (width 1) (layer "B.Cu") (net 15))
 (segment (start 163 64.5) (end 160.5 67) (width 1) (layer "B.Cu") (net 15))
 (segment (start 160.5 67) (end 155.5 67) (width 1) (layer "B.Cu") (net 15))
 (segment (start 157.6925 37.23) (end 157.5 37.0375) (width 1) (layer "B.Cu") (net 32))
 (segment (start 163 37.23) (end 157.6925 37.23) (width 1) (layer "B.Cu") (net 32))
 (segment (start 130 36) (end 120 36) (width 1) (layer "B.Cu") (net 37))
 (segment (start 111.05 44.95) (end 111.05 69.55) (width 1) (layer "B.Cu") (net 37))
 (segment (start 131.08 38.5) (end 131.08 37.08) (width 1) (layer "B.Cu") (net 37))
 (segment (start 120 36) (end 111.05 44.95) (width 1) (layer "B.Cu") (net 37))
 (segment (start 111.05 69.55) (end 111.5 70) (width 1) (layer "B.Cu") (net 37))
 (segment (start 131.08 37.08) (end 130 36) (width 1) (layer "B.Cu") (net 37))
 (segment (start 111.5 70) (end 113.5 70) (width 1) (layer "B.Cu") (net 37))
 (segment (start 117.96 41.46) (end 120.92 38.5) (width 1) (layer "B.Cu") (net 36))
 (segment (start 117.96 44.5) (end 117.96 41.46) (width 1) (layer "B.Cu") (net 36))
 (segment (start 158.35 77.65) (end 158.35 78.62) (width 1) (layer "B.Cu") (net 30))
 (segment (start 164.29 76.5) (end 159.5 76.5) (width 1) (layer "B.Cu") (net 30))
 (segment (start 159.5 76.5) (end 158.35 77.65) (width 1) (layer "B.Cu") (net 30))
 (segment (start 167.77 73.02) (end 164.29 76.5) (width 1) (layer "B.Cu") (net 30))
 (segment (start 165.23 73.02) (end 159.98 73.02) (width 1) (layer "B.Cu") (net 31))
 (segment (start 159.98 73.02) (end 155.81 77.19) (width 1) (layer "B.Cu") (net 31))
 (segment (start 155.81 77.19) (end 155.81 78.62) (width 1) (layer "B.Cu") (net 31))
 (segment (start 167.77 64.02) (end 167.77 66.115) (width 1) (layer "B.Cu") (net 35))
 (segment (start 153.27 75.73) (end 153.27 78.62) (width 1) (layer "B.Cu") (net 35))
 (segment (start 158 71) (end 153.27 75.73) (width 1) (layer "B.Cu") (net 35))
 (segment (start 167.77 66.115) (end 162.885 71) (width 1) (layer "B.Cu") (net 35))
 (segment (start 162.885 71) (end 158 71) (width 1) (layer "B.Cu") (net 35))
 (segment (start 165.23 65.77) (end 162.5 68.5) (width 1) (layer "B.Cu") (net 34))
 (segment (start 165.23 64.02) (end 165.23 65.77) (width 1) (layer "B.Cu") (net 34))
 (segment (start 162.5 68.5) (end 157 68.5) (width 1) (layer "B.Cu") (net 34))
 (segment (start 150.73 74.77) (end 150.73 78.62) (width 1) (layer "B.Cu") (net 34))
 (segment (start 157 68.5) (end 150.73 74.77) (width 1) (layer "B.Cu") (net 34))
 (segment (start 137.28 68.28) (end 143.11 74.11) (width 1) (layer "B.Cu") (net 33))
 (segment (start 137.28 65.5) (end 137.28 68.28) (width 1) (layer "B.Cu") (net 33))
 (segment (start 143.11 74.11) (end 143.11 78.62) (width 1) (layer "B.Cu") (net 33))
 (segment (start 159.6025 39.9625) (end 157.5 39.9625) (width 1) (layer "B.Cu") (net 16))
 (segment (start 162.51 42.87) (end 159.6025 39.9625) (width 1) (layer "B.Cu") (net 16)))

